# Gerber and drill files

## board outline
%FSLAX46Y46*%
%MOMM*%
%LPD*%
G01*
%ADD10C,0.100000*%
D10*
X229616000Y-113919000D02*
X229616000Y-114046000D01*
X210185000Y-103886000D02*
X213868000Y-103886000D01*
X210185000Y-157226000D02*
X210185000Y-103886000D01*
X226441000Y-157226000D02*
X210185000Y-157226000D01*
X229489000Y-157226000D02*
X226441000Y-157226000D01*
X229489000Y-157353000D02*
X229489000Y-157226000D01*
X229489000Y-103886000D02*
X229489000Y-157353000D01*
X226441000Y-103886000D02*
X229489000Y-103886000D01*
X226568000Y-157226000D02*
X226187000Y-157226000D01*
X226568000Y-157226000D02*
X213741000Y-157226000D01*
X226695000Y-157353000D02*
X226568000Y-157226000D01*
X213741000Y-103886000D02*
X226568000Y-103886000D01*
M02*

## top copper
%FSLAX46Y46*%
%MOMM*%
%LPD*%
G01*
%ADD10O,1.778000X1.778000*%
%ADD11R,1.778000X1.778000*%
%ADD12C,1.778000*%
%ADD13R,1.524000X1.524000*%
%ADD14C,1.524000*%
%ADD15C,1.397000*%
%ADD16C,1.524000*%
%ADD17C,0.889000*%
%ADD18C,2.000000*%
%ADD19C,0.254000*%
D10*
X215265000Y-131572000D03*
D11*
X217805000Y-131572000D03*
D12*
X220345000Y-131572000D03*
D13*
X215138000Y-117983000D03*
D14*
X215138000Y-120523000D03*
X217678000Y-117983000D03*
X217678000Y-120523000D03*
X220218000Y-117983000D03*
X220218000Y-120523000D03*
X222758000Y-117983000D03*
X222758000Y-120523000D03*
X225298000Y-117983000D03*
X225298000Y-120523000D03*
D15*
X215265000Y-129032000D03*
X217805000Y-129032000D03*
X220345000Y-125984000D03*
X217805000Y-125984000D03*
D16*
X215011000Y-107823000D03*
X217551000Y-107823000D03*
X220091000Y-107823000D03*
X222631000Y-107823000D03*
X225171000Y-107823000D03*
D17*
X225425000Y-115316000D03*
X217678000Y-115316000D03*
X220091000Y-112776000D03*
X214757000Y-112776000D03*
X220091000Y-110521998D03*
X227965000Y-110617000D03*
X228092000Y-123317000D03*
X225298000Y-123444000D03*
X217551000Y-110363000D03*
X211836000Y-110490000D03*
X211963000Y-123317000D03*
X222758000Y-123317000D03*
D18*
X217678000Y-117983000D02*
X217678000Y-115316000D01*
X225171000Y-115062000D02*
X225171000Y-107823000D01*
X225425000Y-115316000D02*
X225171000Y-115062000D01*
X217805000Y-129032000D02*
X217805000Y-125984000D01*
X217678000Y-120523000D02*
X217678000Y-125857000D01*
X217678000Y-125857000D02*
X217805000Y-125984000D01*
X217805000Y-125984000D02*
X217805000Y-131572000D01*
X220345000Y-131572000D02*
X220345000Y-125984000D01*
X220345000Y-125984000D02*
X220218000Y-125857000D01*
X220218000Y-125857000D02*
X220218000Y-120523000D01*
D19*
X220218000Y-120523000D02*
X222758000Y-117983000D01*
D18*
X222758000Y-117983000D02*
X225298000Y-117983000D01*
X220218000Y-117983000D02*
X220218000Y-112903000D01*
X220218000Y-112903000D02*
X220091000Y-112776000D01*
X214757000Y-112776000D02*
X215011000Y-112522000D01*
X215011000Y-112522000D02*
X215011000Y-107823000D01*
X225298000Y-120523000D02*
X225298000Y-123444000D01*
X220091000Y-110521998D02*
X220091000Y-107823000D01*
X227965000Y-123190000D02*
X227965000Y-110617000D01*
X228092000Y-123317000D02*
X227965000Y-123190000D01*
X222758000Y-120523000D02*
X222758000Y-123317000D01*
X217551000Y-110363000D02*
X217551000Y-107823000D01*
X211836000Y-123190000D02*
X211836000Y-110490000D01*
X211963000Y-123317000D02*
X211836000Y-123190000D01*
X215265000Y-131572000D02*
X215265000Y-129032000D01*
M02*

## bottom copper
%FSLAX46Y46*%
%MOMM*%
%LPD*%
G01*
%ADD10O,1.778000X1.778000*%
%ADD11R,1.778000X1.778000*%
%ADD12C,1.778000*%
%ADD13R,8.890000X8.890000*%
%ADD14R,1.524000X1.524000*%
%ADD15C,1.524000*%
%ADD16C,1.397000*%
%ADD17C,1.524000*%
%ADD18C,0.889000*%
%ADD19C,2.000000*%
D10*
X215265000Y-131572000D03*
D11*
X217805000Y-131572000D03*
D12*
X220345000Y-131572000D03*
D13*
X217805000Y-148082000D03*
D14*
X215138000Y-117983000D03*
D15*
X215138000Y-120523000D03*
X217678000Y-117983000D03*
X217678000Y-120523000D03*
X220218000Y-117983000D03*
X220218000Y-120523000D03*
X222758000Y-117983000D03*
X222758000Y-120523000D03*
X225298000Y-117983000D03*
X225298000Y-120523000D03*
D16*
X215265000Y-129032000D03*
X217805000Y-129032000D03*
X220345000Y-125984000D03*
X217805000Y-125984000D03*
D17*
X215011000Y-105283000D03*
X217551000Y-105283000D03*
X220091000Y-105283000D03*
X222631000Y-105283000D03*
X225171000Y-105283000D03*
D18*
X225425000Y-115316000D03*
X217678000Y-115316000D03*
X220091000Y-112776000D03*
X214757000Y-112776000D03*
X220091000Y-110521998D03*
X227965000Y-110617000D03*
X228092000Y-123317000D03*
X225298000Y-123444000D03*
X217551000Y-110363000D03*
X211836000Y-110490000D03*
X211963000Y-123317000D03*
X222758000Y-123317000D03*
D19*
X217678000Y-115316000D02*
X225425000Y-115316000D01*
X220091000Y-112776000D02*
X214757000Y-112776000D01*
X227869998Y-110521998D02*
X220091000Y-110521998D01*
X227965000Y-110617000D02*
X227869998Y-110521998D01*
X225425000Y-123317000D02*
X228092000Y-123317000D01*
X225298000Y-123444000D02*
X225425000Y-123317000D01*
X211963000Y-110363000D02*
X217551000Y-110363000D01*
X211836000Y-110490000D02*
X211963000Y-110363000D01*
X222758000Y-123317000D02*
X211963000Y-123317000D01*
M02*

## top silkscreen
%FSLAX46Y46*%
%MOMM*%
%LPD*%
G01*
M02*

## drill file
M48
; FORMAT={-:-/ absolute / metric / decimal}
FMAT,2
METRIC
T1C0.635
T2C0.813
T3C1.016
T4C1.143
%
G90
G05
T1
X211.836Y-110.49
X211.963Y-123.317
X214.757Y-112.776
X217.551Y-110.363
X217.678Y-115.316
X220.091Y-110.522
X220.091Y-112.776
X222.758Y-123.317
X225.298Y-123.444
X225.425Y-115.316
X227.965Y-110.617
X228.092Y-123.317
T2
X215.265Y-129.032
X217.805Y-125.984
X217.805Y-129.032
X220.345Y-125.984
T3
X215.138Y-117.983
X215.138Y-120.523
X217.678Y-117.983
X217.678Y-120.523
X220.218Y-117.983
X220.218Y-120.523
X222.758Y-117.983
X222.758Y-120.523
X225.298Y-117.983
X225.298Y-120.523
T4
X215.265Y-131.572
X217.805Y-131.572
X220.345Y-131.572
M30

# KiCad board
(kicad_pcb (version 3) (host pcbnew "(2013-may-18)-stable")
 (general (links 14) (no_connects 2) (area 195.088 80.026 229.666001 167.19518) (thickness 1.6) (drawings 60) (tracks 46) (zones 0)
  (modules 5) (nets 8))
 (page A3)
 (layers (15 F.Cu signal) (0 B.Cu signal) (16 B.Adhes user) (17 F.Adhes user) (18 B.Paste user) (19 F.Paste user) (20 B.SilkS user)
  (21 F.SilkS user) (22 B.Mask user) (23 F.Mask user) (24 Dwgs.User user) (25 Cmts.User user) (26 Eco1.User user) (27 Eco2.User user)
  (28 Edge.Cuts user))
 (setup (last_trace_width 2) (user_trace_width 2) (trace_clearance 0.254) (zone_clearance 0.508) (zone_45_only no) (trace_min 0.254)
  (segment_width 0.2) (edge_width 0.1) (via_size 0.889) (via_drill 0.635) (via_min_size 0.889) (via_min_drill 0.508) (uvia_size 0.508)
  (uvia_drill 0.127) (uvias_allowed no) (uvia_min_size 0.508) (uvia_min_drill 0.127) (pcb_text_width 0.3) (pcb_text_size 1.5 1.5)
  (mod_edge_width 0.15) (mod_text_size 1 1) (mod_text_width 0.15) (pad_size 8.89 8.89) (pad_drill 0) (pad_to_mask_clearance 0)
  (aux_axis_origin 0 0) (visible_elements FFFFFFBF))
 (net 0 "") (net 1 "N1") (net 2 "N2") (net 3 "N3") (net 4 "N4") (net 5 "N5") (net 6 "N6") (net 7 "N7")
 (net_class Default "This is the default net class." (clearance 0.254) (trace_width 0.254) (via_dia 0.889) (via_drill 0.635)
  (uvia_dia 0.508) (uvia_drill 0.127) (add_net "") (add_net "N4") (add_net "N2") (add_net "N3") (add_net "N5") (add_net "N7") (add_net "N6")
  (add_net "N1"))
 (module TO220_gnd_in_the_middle (layer B.Cu) (at 217.805 131.572 270)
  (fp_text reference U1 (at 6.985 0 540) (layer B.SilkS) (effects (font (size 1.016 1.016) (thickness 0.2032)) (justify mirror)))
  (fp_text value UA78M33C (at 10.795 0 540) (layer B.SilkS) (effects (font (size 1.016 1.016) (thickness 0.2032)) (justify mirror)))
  (pad 1 thru_hole oval (at 0 2.54 270) (size 1.778 1.778) (drill 1.143) (layers *.Cu *.Mask B.SilkS) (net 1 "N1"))
  (pad 2 thru_hole rect (at 0 0 270) (size 1.778 1.778) (drill 1.143) (layers *.Cu *.Mask B.SilkS) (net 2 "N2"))
  (pad 3 thru_hole circle (at 0 -2.54 270) (size 1.778 1.778) (drill 1.143) (layers *.Cu *.Mask B.SilkS) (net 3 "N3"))
  (pad 4 smd rect (at 16.51 0 270) (size 8.89 8.89) (layers B.Cu B.Paste B.Mask)))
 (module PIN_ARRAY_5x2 (layer B.Cu) (at 220.218 119.253)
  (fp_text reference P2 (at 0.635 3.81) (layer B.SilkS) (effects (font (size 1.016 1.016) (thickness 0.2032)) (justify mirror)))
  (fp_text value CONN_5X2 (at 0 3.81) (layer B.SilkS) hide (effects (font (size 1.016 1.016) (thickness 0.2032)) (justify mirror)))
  (pad 1 thru_hole rect (at -5.08 -1.27) (size 1.524 1.524) (drill 1.016) (layers *.Cu *.Mask B.SilkS))
  (pad 2 thru_hole circle (at -5.08 1.27) (size 1.524 1.524) (drill 1.016) (layers *.Cu *.Mask B.SilkS))
  (pad 3 thru_hole circle (at -2.54 -1.27) (size 1.524 1.524) (drill 1.016) (layers *.Cu *.Mask B.SilkS) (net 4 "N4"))
  (pad 4 thru_hole circle (at -2.54 1.27) (size 1.524 1.524) (drill 1.016) (layers *.Cu *.Mask B.SilkS) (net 2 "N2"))
  (pad 5 thru_hole circle (at 0 -1.27) (size 1.524 1.524) (drill 1.016) (layers *.Cu *.Mask B.SilkS) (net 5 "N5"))
  (pad 6 thru_hole circle (at 0 1.27) (size 1.524 1.524) (drill 1.016) (layers *.Cu *.Mask B.SilkS) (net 3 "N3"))
  (pad 7 thru_hole circle (at 2.54 -1.27) (size 1.524 1.524) (drill 1.016) (layers *.Cu *.Mask B.SilkS) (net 3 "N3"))
  (pad 8 thru_hole circle (at 2.54 1.27) (size 1.524 1.524) (drill 1.016) (layers *.Cu *.Mask B.SilkS) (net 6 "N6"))
  (pad 9 thru_hole circle (at 5.08 -1.27) (size 1.524 1.524) (drill 1.016) (layers *.Cu *.Mask B.SilkS) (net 3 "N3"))
  (pad 10 thru_hole circle (at 5.08 1.27) (size 1.524 1.524) (drill 1.016) (layers *.Cu *.Mask B.SilkS) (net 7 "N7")))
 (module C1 (layer B.Cu) (at 216.535 129.032)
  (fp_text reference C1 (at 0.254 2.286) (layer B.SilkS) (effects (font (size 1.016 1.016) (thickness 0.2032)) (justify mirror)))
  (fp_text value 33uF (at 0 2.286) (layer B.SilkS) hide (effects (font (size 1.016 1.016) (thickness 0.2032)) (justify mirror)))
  (pad 1 thru_hole circle (at -1.27 0) (size 1.397 1.397) (drill 0.8128) (layers *.Cu *.Mask B.SilkS) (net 1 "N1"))
  (pad 2 thru_hole circle (at 1.27 0) (size 1.397 1.397) (drill 0.8128) (layers *.Cu *.Mask B.SilkS) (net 2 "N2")))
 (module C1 (layer B.Cu) (at 219.075 125.984 180)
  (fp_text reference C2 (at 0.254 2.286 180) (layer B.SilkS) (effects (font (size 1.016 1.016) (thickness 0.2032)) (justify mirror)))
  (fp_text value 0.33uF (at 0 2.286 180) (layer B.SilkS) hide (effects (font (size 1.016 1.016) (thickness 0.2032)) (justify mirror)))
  (pad 1 thru_hole circle (at -1.27 0 180) (size 1.397 1.397) (drill 0.8128) (layers *.Cu *.Mask B.SilkS) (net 3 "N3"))
  (pad 2 thru_hole circle (at 1.27 0 180) (size 1.397 1.397) (drill 0.8128) (layers *.Cu *.Mask B.SilkS) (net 2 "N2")))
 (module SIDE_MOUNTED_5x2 (layer B.Cu) (at 220.091 106.553)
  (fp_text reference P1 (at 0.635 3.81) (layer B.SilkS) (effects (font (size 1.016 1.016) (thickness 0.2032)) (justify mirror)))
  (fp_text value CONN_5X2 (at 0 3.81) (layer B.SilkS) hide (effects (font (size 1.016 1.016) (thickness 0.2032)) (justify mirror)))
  (pad 1 smd circle (at -5.08 -1.27) (size 1.524 1.524) (layers B.Cu B.Paste B.Mask) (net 2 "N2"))
  (pad 2 smd circle (at -5.08 1.27) (size 1.524 1.524) (layers F.Cu B.Paste B.Mask) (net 5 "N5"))
  (pad 3 smd circle (at -2.54 -1.27) (size 1.524 1.524) (layers B.Cu B.Paste B.Mask) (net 1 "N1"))
  (pad 4 smd circle (at -2.54 1.27) (size 1.524 1.524) (layers F.Cu B.Paste B.Mask) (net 6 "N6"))
  (pad 5 smd circle (at 0 -1.27) (size 1.524 1.524) (layers B.Cu B.Paste B.Mask))
  (pad 6 smd circle (at 0 1.27) (size 1.524 1.524) (layers F.Cu B.Paste B.Mask) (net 7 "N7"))
  (pad 7 smd circle (at 2.54 -1.27) (size 1.524 1.524) (layers B.Cu B.Paste B.Mask))
  (pad 8 smd circle (at 2.54 1.27) (size 1.524 1.524) (layers F.Cu B.Paste B.Mask))
  (pad 9 smd circle (at 5.08 -1.27) (size 1.524 1.524) (layers B.Cu B.Paste B.Mask))
  (pad 10 smd circle (at 5.08 1.27) (size 1.524 1.524) (layers F.Cu B.Paste B.Mask) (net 4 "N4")))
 (gr_line (start 229.616 113.919) (end 229.616 114.046) (angle 90) (layer Edge.Cuts) (width 0.1))
 (gr_line (start 210.185 103.886) (end 213.868 103.886) (angle 90) (layer Edge.Cuts) (width 0.1))
 (gr_line (start 210.185 157.226) (end 210.185 103.886) (angle 90) (layer Edge.Cuts) (width 0.1))
 (gr_line (start 226.441 157.226) (end 210.185 157.226) (angle 90) (layer Edge.Cuts) (width 0.1))
 (gr_line (start 229.489 157.226) (end 226.441 157.226) (angle 90) (layer Edge.Cuts) (width 0.1))
 (gr_line (start 229.489 157.353) (end 229.489 157.226) (angle 90) (layer Edge.Cuts) (width 0.1))
 (gr_line (start 229.489 103.886) (end 229.489 157.353) (angle 90) (layer Edge.Cuts) (width 0.1))
 (gr_line (start 226.441 103.886) (end 229.489 103.886) (angle 90) (layer Edge.Cuts) (width 0.1))
 (gr_line (start 226.568 157.226) (end 226.187 157.226) (angle 90) (layer Edge.Cuts) (width 0.1))
 (gr_line (start 226.568 157.226) (end 213.741 157.226) (angle 90) (layer Edge.Cuts) (width 0.1))
 (gr_line (start 226.695 157.353) (end 226.568 157.226) (angle 90) (layer Edge.Cuts) (width 0.1))
 (gr_line (start 213.741 103.886) (end 226.568 103.886) (angle 90) (layer Edge.Cuts) (width 0.1))
 (segment (start 217.678 117.983) (end 217.678 115.316) (width 2) (layer F.Cu) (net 4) (status 400000))
 (segment (start 225.171 115.062) (end 225.171 107.823) (width 2) (layer F.Cu) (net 4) (status 800000))
 (segment (start 225.425 115.316) (end 225.171 115.062) (width 2) (layer F.Cu) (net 4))
 (via (at 225.425 115.316) (size 0.889) (layers F.Cu B.Cu) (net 4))
 (segment (start 217.678 115.316) (end 225.425 115.316) (width 2) (layer B.Cu) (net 4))
 (via (at 217.678 115.316) (size 0.889) (layers F.Cu B.Cu) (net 4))
 (segment (start 217.805 129.032) (end 217.805 125.984) (width 2) (layer F.Cu) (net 2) (status C00000))
 (segment (start 217.678 120.523) (end 217.678 125.857) (width 2) (layer F.Cu) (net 2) (status C00000))
 (segment (start 217.678 125.857) (end 217.805 125.984) (width 2) (layer F.Cu) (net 2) (status C00000))
 (segment (start 217.805 125.984) (end 217.805 131.572) (width 2) (layer F.Cu) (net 2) (status C00000))
 (segment (start 220.345 131.572) (end 220.345 125.984) (width 2) (layer F.Cu) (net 3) (status C00000))
 (segment (start 220.345 125.984) (end 220.218 125.857) (width 2) (layer F.Cu) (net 3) (status C00000))
 (segment (start 220.218 125.857) (end 220.218 120.523) (width 2) (layer F.Cu) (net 3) (status C00000))
 (segment (start 220.218 120.523) (end 222.758 117.983) (width 0.254) (layer F.Cu) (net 3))
 (segment (start 222.758 117.983) (end 225.298 117.983) (width 2) (layer F.Cu) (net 3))
 (segment (start 220.218 117.983) (end 220.218 112.903) (width 2) (layer F.Cu) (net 5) (status 400000))
 (segment (start 220.218 112.903) (end 220.091 112.776) (width 2) (layer F.Cu) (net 5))
 (via (at 220.091 112.776) (size 0.889) (layers F.Cu B.Cu) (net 5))
 (segment (start 220.091 112.776) (end 214.757 112.776) (width 2) (layer B.Cu) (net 5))
 (via (at 214.757 112.776) (size 0.889) (layers F.Cu B.Cu) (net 5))
 (segment (start 214.757 112.776) (end 215.011 112.522) (width 2) (layer F.Cu) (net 5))
 (segment (start 215.011 112.522) (end 215.011 107.823) (width 2) (layer F.Cu) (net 5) (status 800000))
 (segment (start 225.298 120.523) (end 225.298 123.444) (width 2) (layer F.Cu) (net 7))
 (segment (start 220.091 110.521998) (end 220.091 107.823) (width 2) (layer F.Cu) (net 7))
 (via (at 220.091 110.521998) (size 0.889) (layers F.Cu B.Cu) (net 7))
 (segment (start 227.869998 110.521998) (end 220.091 110.521998) (width 2) (layer B.Cu) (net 7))
 (segment (start 227.965 110.617) (end 227.869998 110.521998) (width 2) (layer B.Cu) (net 7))
 (via (at 227.965 110.617) (size 0.889) (layers F.Cu B.Cu) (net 7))
 (segment (start 227.965 123.19) (end 227.965 110.617) (width 2) (layer F.Cu) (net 7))
 (segment (start 228.092 123.317) (end 227.965 123.19) (width 2) (layer F.Cu) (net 7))
 (via (at 228.092 123.317) (size 0.889) (layers F.Cu B.Cu) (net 7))
 (segment (start 225.425 123.317) (end 228.092 123.317) (width 2) (layer B.Cu) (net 7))
 (segment (start 225.298 123.444) (end 225.425 123.317) (width 2) (layer B.Cu) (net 7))
 (via (at 225.298 123.444) (size 0.889) (layers F.Cu B.Cu) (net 7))
 (segment (start 222.758 120.523) (end 222.758 123.317) (width 2) (layer F.Cu) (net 6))
 (segment (start 217.551 110.363) (end 217.551 107.823) (width 2) (layer F.Cu) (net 6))
 (via (at 217.551 110.363) (size 0.889) (layers F.Cu B.Cu) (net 6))
 (segment (start 211.963 110.363) (end 217.551 110.363) (width 2) (layer B.Cu) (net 6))
 (segment (start 211.836 110.49) (end 211.963 110.363) (width 2) (layer B.Cu) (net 6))
 (via (at 211.836 110.49) (size 0.889) (layers F.Cu B.Cu) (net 6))
 (segment (start 211.836 123.19) (end 211.836 110.49) (width 2) (layer F.Cu) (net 6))
 (segment (start 211.963 123.317) (end 211.836 123.19) (width 2) (layer F.Cu) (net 6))
 (via (at 211.963 123.317) (size 0.889) (layers F.Cu B.Cu) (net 6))
 (segment (start 222.758 123.317) (end 211.963 123.317) (width 2) (layer B.Cu) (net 6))
 (via (at 222.758 123.317) (size 0.889) (layers F.Cu B.Cu) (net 6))
 (segment (start 215.265 131.572) (end 215.265 129.032) (width 2) (layer F.Cu) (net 1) (status C00000)))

